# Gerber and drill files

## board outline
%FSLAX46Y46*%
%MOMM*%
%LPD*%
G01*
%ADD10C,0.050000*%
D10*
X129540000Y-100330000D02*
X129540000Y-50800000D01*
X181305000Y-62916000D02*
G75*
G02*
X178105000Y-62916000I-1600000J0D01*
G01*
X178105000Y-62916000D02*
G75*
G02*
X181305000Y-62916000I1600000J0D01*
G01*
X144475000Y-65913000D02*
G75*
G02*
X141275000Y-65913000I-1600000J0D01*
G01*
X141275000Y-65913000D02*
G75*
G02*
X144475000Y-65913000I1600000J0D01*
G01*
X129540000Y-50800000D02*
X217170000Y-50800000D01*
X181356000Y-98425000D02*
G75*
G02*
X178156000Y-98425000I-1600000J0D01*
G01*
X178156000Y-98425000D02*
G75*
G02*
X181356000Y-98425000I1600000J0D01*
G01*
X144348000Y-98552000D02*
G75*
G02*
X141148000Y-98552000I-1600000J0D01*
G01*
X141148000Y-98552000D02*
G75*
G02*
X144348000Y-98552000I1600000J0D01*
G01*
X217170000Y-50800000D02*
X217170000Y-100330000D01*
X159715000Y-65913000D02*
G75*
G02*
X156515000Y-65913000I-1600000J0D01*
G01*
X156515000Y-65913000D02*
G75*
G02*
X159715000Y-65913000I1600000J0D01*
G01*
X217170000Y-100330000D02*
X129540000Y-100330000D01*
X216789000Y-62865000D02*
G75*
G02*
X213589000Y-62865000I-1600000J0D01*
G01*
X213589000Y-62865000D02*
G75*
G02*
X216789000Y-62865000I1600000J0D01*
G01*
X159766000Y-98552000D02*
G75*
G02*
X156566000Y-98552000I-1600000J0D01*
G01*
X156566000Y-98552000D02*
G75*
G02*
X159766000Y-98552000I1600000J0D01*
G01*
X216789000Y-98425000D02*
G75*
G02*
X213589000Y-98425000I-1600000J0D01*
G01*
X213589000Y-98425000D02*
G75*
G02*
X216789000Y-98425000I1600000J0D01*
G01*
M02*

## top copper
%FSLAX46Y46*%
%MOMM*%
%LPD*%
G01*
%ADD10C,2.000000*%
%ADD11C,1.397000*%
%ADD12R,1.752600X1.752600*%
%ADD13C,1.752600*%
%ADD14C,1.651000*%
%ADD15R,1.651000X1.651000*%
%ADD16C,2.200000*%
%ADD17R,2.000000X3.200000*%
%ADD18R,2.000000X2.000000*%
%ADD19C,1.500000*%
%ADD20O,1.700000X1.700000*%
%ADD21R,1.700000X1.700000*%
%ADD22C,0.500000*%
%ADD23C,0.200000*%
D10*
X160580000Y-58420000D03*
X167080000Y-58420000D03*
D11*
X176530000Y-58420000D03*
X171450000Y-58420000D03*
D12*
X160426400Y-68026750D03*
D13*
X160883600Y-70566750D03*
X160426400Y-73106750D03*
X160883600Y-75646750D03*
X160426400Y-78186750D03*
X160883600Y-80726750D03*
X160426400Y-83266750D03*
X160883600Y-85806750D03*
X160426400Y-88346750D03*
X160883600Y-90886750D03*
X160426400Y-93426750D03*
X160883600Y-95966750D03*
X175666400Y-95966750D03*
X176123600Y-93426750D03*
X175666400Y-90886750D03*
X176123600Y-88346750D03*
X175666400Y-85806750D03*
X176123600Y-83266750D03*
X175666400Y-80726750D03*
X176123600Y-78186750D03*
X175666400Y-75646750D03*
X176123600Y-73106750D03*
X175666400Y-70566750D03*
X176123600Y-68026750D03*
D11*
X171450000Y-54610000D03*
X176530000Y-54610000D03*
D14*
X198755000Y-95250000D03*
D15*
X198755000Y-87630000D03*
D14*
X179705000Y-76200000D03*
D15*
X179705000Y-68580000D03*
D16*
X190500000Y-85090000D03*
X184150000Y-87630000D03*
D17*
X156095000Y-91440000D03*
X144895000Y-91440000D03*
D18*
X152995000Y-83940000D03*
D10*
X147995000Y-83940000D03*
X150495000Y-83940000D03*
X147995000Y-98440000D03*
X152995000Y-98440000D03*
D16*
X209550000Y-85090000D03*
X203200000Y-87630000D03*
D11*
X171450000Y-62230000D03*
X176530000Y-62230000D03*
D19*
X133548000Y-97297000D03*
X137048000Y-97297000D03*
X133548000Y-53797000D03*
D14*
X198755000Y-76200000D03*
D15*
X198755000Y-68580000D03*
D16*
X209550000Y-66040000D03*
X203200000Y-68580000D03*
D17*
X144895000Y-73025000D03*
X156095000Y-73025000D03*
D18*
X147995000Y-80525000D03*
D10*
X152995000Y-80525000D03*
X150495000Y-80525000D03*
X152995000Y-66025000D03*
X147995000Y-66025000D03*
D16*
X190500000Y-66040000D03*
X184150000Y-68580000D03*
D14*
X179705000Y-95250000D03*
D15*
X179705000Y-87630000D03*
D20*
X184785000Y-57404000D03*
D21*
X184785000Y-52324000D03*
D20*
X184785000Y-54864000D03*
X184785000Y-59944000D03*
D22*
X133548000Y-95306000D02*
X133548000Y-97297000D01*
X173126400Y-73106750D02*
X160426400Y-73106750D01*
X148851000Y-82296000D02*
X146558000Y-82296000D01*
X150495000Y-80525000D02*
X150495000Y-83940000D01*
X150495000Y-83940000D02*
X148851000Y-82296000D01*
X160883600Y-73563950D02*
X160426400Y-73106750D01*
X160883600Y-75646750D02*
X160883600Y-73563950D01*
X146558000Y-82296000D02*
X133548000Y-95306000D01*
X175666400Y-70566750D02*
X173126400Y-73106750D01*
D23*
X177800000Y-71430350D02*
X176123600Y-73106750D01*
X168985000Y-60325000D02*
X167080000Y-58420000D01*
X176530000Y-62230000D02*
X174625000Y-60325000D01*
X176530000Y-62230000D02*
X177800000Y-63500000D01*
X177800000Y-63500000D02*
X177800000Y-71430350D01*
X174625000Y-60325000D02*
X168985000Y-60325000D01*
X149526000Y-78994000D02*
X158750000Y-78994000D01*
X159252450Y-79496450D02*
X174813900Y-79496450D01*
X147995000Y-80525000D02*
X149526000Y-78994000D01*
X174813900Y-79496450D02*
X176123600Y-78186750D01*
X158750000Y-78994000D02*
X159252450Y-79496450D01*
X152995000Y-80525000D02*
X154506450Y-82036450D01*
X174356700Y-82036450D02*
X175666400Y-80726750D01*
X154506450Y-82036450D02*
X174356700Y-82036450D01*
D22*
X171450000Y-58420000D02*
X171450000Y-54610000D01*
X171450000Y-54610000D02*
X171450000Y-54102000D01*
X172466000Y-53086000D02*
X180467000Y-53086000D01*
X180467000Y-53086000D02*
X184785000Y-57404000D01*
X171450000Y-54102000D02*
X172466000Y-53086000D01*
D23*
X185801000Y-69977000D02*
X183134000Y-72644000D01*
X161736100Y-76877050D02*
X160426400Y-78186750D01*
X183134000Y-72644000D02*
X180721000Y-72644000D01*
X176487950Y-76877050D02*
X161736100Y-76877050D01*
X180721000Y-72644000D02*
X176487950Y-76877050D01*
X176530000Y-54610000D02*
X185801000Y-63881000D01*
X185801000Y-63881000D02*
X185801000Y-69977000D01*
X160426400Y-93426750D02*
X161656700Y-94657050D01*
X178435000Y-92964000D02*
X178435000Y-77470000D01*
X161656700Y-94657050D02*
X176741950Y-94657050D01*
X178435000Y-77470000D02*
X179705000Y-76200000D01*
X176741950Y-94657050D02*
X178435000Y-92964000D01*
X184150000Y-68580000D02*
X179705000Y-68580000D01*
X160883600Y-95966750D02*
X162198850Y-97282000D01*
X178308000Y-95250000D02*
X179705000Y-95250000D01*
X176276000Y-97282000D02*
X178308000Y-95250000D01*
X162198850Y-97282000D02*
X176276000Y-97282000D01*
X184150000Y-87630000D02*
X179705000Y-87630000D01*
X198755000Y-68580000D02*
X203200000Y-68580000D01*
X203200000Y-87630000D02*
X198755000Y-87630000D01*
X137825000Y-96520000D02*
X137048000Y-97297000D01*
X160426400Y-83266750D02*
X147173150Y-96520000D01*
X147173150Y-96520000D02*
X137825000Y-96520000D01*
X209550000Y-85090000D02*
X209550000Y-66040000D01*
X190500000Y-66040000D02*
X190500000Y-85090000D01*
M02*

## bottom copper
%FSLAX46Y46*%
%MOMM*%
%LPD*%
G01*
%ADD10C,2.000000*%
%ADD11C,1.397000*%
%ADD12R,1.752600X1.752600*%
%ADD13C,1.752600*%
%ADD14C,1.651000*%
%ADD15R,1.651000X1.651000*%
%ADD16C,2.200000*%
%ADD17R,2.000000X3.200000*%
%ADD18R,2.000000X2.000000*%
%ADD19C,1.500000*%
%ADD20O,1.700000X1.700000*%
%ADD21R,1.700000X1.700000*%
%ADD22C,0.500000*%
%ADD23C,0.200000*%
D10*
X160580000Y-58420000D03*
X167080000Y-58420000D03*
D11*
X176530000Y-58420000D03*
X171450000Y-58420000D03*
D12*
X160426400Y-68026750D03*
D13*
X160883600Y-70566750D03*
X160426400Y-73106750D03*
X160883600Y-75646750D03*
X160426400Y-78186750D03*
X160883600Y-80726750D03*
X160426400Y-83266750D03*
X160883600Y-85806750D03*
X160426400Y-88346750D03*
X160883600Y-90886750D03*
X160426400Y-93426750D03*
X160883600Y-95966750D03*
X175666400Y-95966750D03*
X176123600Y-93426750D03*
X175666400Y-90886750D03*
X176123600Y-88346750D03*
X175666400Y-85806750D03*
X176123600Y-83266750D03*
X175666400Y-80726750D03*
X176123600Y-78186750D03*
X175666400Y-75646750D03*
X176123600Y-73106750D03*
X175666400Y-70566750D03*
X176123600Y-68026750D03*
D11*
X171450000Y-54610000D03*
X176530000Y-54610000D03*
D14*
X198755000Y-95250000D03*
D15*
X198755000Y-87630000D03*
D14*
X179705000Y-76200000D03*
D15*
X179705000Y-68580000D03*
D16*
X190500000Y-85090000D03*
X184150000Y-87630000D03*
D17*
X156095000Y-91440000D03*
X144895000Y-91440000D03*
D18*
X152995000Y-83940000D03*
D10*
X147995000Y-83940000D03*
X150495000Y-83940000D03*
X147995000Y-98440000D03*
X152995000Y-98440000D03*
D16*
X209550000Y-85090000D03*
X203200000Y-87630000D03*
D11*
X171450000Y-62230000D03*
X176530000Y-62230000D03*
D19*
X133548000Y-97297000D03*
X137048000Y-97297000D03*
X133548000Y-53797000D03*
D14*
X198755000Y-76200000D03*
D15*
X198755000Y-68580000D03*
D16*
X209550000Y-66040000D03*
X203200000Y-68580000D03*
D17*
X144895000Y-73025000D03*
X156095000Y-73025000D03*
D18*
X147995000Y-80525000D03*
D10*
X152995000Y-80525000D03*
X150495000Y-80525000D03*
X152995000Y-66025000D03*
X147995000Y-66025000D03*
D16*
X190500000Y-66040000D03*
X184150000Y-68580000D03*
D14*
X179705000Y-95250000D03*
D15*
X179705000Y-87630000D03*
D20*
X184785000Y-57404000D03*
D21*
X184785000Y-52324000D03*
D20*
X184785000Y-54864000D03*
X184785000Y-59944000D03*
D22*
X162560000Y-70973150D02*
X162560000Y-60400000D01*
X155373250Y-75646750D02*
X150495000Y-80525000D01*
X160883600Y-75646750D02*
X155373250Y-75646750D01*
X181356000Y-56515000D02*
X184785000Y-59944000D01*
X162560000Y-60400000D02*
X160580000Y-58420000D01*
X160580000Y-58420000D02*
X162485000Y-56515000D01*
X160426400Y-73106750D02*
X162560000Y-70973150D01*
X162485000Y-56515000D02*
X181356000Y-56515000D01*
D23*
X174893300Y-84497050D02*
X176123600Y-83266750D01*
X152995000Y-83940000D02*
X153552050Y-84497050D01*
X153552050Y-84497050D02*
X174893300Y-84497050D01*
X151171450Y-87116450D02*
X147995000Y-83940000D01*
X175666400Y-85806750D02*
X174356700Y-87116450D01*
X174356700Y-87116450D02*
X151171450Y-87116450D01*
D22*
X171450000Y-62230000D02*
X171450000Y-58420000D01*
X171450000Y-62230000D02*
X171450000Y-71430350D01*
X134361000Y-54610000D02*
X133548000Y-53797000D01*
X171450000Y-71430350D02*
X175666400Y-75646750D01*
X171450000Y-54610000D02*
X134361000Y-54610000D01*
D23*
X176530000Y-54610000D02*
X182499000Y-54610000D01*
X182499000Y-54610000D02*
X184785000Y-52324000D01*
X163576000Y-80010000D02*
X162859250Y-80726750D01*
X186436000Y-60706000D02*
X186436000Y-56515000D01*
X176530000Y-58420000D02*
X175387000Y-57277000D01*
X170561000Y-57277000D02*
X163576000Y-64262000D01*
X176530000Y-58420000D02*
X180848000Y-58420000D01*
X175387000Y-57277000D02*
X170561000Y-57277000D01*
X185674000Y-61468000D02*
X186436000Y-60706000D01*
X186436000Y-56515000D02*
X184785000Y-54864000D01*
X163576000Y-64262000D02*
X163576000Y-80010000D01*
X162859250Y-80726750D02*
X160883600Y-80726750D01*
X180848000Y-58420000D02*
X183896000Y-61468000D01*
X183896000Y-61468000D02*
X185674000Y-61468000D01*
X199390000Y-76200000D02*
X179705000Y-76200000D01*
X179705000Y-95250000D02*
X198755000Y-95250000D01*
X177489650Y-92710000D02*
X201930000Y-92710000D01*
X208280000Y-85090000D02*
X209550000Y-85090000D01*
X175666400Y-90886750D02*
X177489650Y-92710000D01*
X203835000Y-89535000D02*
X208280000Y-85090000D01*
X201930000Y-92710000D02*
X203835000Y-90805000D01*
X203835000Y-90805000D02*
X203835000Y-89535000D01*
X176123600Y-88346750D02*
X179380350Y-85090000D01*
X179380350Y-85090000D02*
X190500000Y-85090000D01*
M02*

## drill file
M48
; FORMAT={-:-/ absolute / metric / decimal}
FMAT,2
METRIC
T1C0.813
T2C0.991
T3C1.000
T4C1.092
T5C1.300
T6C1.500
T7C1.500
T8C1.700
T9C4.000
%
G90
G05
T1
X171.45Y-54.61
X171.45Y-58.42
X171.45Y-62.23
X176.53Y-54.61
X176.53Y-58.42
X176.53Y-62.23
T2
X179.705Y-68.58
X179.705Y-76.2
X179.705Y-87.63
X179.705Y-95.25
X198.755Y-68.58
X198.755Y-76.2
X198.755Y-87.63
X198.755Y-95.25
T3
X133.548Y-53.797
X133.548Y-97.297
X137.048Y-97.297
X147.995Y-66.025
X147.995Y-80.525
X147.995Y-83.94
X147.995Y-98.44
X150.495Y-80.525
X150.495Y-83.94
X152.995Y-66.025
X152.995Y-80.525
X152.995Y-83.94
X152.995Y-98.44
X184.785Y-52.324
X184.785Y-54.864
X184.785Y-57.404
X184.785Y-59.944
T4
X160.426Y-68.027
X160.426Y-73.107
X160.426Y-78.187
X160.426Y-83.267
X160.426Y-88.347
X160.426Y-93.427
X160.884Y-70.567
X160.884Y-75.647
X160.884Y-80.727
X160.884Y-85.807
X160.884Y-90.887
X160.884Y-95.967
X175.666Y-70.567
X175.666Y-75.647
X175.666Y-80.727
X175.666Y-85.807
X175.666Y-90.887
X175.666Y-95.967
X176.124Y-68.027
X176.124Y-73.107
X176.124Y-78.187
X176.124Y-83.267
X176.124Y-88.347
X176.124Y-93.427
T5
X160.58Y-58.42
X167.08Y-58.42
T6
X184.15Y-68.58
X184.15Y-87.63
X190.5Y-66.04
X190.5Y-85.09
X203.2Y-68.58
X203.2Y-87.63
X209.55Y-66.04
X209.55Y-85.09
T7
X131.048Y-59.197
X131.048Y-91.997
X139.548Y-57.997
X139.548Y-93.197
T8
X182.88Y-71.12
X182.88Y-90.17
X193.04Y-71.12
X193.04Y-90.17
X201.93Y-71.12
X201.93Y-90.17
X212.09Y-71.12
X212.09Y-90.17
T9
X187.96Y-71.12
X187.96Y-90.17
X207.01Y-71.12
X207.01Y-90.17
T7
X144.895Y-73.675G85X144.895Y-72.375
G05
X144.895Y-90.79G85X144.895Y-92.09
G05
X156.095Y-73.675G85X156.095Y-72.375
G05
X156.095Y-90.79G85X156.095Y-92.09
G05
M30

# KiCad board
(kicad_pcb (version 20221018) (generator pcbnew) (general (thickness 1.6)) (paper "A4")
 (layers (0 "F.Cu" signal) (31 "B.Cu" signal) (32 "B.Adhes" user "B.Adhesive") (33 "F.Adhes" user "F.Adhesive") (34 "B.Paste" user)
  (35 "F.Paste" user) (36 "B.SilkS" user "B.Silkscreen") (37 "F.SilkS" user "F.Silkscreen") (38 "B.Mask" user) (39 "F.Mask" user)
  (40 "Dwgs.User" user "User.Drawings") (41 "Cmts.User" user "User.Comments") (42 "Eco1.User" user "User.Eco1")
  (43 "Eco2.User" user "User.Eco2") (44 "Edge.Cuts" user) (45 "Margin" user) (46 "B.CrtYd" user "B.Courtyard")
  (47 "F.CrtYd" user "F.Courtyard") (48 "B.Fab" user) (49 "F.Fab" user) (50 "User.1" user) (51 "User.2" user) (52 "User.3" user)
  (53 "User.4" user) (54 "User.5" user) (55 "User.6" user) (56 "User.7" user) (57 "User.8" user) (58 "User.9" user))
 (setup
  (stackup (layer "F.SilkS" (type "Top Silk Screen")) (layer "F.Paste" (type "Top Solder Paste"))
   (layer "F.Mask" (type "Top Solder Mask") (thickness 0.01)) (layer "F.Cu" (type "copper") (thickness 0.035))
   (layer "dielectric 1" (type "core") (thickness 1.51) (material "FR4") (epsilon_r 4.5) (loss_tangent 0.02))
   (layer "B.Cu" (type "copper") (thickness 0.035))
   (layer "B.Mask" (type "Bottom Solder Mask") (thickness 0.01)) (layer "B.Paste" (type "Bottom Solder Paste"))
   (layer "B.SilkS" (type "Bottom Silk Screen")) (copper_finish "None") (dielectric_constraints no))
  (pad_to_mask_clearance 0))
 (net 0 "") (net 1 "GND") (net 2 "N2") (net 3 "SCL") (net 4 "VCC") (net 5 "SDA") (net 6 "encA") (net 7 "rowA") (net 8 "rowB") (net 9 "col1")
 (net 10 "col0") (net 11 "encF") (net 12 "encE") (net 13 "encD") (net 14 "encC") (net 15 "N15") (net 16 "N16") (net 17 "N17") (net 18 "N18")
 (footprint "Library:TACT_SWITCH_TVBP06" (layer "F.Cu") (at 163.83 58.42)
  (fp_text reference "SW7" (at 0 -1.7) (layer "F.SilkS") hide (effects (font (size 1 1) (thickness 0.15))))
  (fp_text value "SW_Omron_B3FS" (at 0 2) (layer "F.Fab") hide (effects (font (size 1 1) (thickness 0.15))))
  (pad "1" thru_hole circle (at -3.25 0) (size 2 2) (drill 1.3) (layers "*.Cu" "*.Mask") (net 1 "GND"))
  (pad "2" thru_hole circle (at 3.25 0) (size 2 2) (drill 1.3) (layers "*.Cu" "*.Mask") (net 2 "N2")))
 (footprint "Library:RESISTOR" (layer "F.Cu") (at 173.99 58.42 180)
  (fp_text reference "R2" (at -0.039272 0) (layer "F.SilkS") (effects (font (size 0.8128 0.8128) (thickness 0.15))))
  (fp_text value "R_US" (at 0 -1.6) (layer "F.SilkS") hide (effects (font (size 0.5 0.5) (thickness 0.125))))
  (pad "1" thru_hole circle (at -2.54 0 180) (size 1.397 1.397) (drill 0.8128) (layers "*.Cu" "*.Mask") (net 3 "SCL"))
  (pad "2" thru_hole circle (at 2.54 0 180) (size 1.397 1.397) (drill 0.8128) (layers "*.Cu" "*.Mask") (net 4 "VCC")))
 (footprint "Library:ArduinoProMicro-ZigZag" (layer "F.Cu") (at 168.275 81.99675 -90)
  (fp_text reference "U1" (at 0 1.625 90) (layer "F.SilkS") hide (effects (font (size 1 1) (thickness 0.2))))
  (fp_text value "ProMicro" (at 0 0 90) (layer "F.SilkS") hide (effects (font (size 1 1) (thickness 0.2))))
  (pad "1" thru_hole rect (at -13.97 7.8486 270) (size 1.7526 1.7526) (drill 1.0922) (layers "*.Cu" "*.SilkS" "*.Mask"))
  (pad "2" thru_hole circle (at -11.43 7.3914 270) (size 1.7526 1.7526) (drill 1.0922) (layers "*.Cu" "*.SilkS" "*.Mask"))
  (pad "3" thru_hole circle (at -8.89 7.8486 270) (size 1.7526 1.7526) (drill 1.0922) (layers "*.Cu" "*.SilkS" "*.Mask") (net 1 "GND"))
  (pad "4" thru_hole circle (at -6.35 7.3914 270) (size 1.7526 1.7526) (drill 1.0922) (layers "*.Cu" "*.SilkS" "*.Mask") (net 1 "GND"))
  (pad "5" thru_hole circle (at -3.81 7.8486 270) (size 1.7526 1.7526) (drill 1.0922) (layers "*.Cu" "*.SilkS" "*.Mask") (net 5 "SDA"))
  (pad "6" thru_hole circle (at -1.27 7.3914 270) (size 1.7526 1.7526) (drill 1.0922) (layers "*.Cu" "*.SilkS" "*.Mask") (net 3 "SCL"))
  (pad "7" thru_hole circle (at 1.27 7.8486 270) (size 1.7526 1.7526) (drill 1.0922) (layers "*.Cu" "*.SilkS" "*.Mask") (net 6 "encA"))
  (pad "8" thru_hole circle (at 3.81 7.3914 270) (size 1.7526 1.7526) (drill 1.0922) (layers "*.Cu" "*.SilkS" "*.Mask"))
  (pad "9" thru_hole circle (at 6.35 7.8486 270) (size 1.7526 1.7526) (drill 1.0922) (layers "*.Cu" "*.SilkS" "*.Mask"))
  (pad "10" thru_hole circle (at 8.89 7.3914 270) (size 1.7526 1.7526) (drill 1.0922) (layers "*.Cu" "*.SilkS" "*.Mask"))
  (pad "11" thru_hole circle (at 11.43 7.8486 270) (size 1.7526 1.7526) (drill 1.0922) (layers "*.Cu" "*.SilkS" "*.Mask") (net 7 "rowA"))
  (pad "12" thru_hole circle (at 13.97 7.3914 270) (size 1.7526 1.7526) (drill 1.0922) (layers "*.Cu" "*.SilkS" "*.Mask") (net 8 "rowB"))
  (pad "13" thru_hole circle (at 13.97 -7.3914 270) (size 1.7526 1.7526) (drill 1.0922) (layers "*.Cu" "*.SilkS" "*.Mask"))
  (pad "14" thru_hole circle (at 11.43 -7.8486 270) (size 1.7526 1.7526) (drill 1.0922) (layers "*.Cu" "*.SilkS" "*.Mask"))
  (pad "15" thru_hole circle (at 8.89 -7.3914 270) (size 1.7526 1.7526) (drill 1.0922) (layers "*.Cu" "*.SilkS" "*.Mask") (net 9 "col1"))
  (pad "16" thru_hole circle (at 6.35 -7.8486 270) (size 1.7526 1.7526) (drill 1.0922) (layers "*.Cu" "*.SilkS" "*.Mask") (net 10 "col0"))
  (pad "17" thru_hole circle (at 3.81 -7.3914 270) (size 1.7526 1.7526) (drill 1.0922) (layers "*.Cu" "*.SilkS" "*.Mask") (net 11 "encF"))
  (pad "18" thru_hole circle (at 1.27 -7.8486 270) (size 1.7526 1.7526) (drill 1.0922) (layers "*.Cu" "*.SilkS" "*.Mask") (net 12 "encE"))
  (pad "19" thru_hole circle (at -1.27 -7.3914 270) (size 1.7526 1.7526) (drill 1.0922) (layers "*.Cu" "*.SilkS" "*.Mask") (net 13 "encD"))
  (pad "20" thru_hole circle (at -3.81 -7.8486 270) (size 1.7526 1.7526) (drill 1.0922) (layers "*.Cu" "*.SilkS" "*.Mask") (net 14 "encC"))
  (pad "21" thru_hole circle (at -6.35 -7.3914 270) (size 1.7526 1.7526) (drill 1.0922) (layers "*.Cu" "*.SilkS" "*.Mask") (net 4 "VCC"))
  (pad "22" thru_hole circle (at -8.89 -7.8486 270) (size 1.7526 1.7526) (drill 1.0922) (layers "*.Cu" "*.SilkS" "*.Mask") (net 2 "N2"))
  (pad "23" thru_hole circle (at -11.43 -7.3914 270) (size 1.7526 1.7526) (drill 1.0922) (layers "*.Cu" "*.SilkS" "*.Mask") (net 1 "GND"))
  (pad "24" thru_hole circle (at -13.97 -7.8486 270) (size 1.7526 1.7526) (drill 1.0922) (layers "*.Cu" "*.SilkS" "*.Mask")))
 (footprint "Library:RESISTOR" (layer "F.Cu") (at 173.99 54.61)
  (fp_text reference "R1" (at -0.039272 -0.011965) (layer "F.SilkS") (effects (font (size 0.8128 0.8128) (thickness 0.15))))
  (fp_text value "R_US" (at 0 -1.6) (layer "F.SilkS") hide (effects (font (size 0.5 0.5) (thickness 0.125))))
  (pad "1" thru_hole circle (at -2.54 0) (size 1.397 1.397) (drill 0.8128) (layers "*.Cu" "*.Mask") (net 4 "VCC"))
  (pad "2" thru_hole circle (at 2.54 0) (size 1.397 1.397) (drill 0.8128) (layers "*.Cu" "*.Mask") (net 5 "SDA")))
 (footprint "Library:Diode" (layer "F.Cu") (at 198.755 91.44 90)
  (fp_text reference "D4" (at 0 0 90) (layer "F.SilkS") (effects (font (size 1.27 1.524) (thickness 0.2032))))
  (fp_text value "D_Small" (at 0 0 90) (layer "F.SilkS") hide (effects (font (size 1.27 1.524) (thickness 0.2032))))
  (pad "1" thru_hole circle (at -3.81 0 90) (size 1.651 1.651) (drill 0.9906) (layers "*.Cu" "*.SilkS" "*.Mask") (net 8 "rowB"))
  (pad "2" thru_hole rect (at 3.81 0 90) (size 1.651 1.651) (drill 0.9906) (layers "*.Cu" "*.SilkS" "*.Mask") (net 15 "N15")))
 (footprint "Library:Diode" (layer "F.Cu") (at 179.705 72.39 90)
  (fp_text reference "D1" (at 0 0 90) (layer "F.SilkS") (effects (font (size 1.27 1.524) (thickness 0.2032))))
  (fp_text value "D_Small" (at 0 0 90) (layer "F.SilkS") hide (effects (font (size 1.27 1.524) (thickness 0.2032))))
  (pad "1" thru_hole circle (at -3.81 0 90) (size 1.651 1.651) (drill 0.9906) (layers "*.Cu" "*.SilkS" "*.Mask") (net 7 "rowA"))
  (pad "2" thru_hole rect (at 3.81 0 90) (size 1.651 1.651) (drill 0.9906) (layers "*.Cu" "*.SilkS" "*.Mask") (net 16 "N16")))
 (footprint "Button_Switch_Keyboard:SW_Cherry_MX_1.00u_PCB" (layer "F.Cu") (at 190.5 85.09)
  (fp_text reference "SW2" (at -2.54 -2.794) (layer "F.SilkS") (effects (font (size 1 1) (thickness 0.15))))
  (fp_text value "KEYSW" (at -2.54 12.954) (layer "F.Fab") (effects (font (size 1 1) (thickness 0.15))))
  (pad "" np_thru_hole circle (at -7.62 5.08) (size 1.7 1.7) (drill 1.7) (layers "*.Cu" "*.Mask"))
  (pad "" np_thru_hole circle (at -2.54 5.08) (size 4 4) (drill 4) (layers "*.Cu" "*.Mask"))
  (pad "" np_thru_hole circle (at 2.54 5.08) (size 1.7 1.7) (drill 1.7) (layers "*.Cu" "*.Mask"))
  (pad "1" thru_hole circle (at 0 0) (size 2.2 2.2) (drill 1.5) (layers "*.Cu" "*.Mask") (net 10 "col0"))
  (pad "2" thru_hole circle (at -6.35 2.54) (size 2.2 2.2) (drill 1.5) (layers "*.Cu" "*.Mask") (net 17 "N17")))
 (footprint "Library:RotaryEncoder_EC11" (layer "F.Cu") (at 150.495 91.44 -90)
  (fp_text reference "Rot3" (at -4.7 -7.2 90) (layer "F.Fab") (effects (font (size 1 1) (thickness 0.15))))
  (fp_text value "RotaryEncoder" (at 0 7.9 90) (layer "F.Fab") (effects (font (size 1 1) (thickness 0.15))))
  (pad "" np_thru_hole rect (at 0 -5.6 270) (size 3.2 2) (drill oval 2.8 1.5) (layers "*.Cu" "*.Mask"))
  (pad "" np_thru_hole rect (at 0 5.6 270) (size 3.2 2) (drill oval 2.8 1.5) (layers "*.Cu" "*.Mask"))
  (pad "A" thru_hole rect (at -7.5 -2.5 270) (size 2 2) (drill 1) (layers "*.Cu" "*.Mask") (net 12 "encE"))
  (pad "B" thru_hole circle (at -7.5 2.5 270) (size 2 2) (drill 1) (layers "*.Cu" "*.Mask") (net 11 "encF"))
  (pad "C" thru_hole circle (at -7.5 0 270) (size 2 2) (drill 1) (layers "*.Cu" "*.Mask") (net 1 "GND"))
  (pad "S1" thru_hole circle (at 7 2.5 270) (size 2 2) (drill 1) (layers "*.Cu" "*.Mask"))
  (pad "S2" thru_hole circle (at 7 -2.5 270) (size 2 2) (drill 1) (layers "*.Cu" "*.Mask")))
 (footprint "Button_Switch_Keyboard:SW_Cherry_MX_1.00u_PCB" (layer "F.Cu") (at 209.55 85.09)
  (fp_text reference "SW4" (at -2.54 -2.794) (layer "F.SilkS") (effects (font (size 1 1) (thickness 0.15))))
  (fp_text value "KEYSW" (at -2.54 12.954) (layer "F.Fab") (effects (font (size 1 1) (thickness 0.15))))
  (pad "" np_thru_hole circle (at -7.62 5.08) (size 1.7 1.7) (drill 1.7) (layers "*.Cu" "*.Mask"))
  (pad "" np_thru_hole circle (at -2.54 5.08) (size 4 4) (drill 4) (layers "*.Cu" "*.Mask"))
  (pad "" np_thru_hole circle (at 2.54 5.08) (size 1.7 1.7) (drill 1.7) (layers "*.Cu" "*.Mask"))
  (pad "1" thru_hole circle (at 0 0) (size 2.2 2.2) (drill 1.5) (layers "*.Cu" "*.Mask") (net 9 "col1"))
  (pad "2" thru_hole circle (at -6.35 2.54) (size 2.2 2.2) (drill 1.5) (layers "*.Cu" "*.Mask") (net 15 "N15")))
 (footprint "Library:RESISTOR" (layer "F.Cu") (at 173.99 62.23)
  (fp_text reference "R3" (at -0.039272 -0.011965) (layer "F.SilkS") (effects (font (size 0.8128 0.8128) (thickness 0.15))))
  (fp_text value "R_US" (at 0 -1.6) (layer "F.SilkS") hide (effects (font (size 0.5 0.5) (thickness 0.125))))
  (pad "1" thru_hole circle (at -2.54 0) (size 1.397 1.397) (drill 0.8128) (layers "*.Cu" "*.Mask") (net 4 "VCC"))
  (pad "2" thru_hole circle (at 2.54 0) (size 1.397 1.397) (drill 0.8128) (layers "*.Cu" "*.Mask") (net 2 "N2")))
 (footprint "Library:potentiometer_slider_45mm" (layer "F.Cu") (at 142.248 98.097 90)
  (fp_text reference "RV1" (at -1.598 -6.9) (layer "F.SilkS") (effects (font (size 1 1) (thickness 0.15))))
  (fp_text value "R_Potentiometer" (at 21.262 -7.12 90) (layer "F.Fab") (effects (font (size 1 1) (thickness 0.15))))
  (pad "" np_thru_hole circle (at 4.9 -2.7 90) (size 1.5 1.5) (drill 1.5) (layers "*.Cu" "*.Mask"))
  (pad "" np_thru_hole circle (at 6.1 -11.2 90) (size 1.5 1.5) (drill 1.5) (layers "*.Cu" "*.Mask"))
  (pad "" np_thru_hole circle (at 38.9 -11.2 90) (size 1.5 1.5) (drill 1.5) (layers "*.Cu" "*.Mask"))
  (pad "" np_thru_hole circle (at 40.1 -2.7 90) (size 1.5 1.5) (drill 1.5) (layers "*.Cu" "*.Mask"))
  (pad "1" thru_hole circle (at 0.8 -8.7 90) (size 1.5 1.5) (drill 1) (layers "*.Cu" "*.Mask") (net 1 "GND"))
  (pad "2" thru_hole circle (at 0.8 -5.2 90) (size 1.5 1.5) (drill 1) (layers "*.Cu" "*.Mask") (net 6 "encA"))
  (pad "3" thru_hole circle (at 44.3 -8.7 90) (size 1.5 1.5) (drill 1) (layers "*.Cu" "*.Mask") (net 4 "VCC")))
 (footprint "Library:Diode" (layer "F.Cu") (at 198.755 72.39 90)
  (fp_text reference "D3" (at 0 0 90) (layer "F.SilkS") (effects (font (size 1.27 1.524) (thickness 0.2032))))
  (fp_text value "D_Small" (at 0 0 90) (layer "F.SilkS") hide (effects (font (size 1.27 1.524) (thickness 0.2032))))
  (pad "1" thru_hole circle (at -3.81 0 90) (size 1.651 1.651) (drill 0.9906) (layers "*.Cu" "*.SilkS" "*.Mask") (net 7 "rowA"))
  (pad "2" thru_hole rect (at 3.81 0 90) (size 1.651 1.651) (drill 0.9906) (layers "*.Cu" "*.SilkS" "*.Mask") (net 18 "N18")))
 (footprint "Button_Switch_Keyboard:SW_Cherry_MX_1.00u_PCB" (layer "F.Cu") (at 209.55 66.04)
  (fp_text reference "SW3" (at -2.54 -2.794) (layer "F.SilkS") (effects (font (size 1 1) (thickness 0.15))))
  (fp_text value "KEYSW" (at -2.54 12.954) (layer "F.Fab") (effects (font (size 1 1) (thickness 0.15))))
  (pad "" np_thru_hole circle (at -7.62 5.08) (size 1.7 1.7) (drill 1.7) (layers "*.Cu" "*.Mask"))
  (pad "" np_thru_hole circle (at -2.54 5.08) (size 4 4) (drill 4) (layers "*.Cu" "*.Mask"))
  (pad "" np_thru_hole circle (at 2.54 5.08) (size 1.7 1.7) (drill 1.7) (layers "*.Cu" "*.Mask"))
  (pad "1" thru_hole circle (at 0 0) (size 2.2 2.2) (drill 1.5) (layers "*.Cu" "*.Mask") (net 9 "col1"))
  (pad "2" thru_hole circle (at -6.35 2.54) (size 2.2 2.2) (drill 1.5) (layers "*.Cu" "*.Mask") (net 18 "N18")))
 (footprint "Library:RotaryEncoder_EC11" (layer "F.Cu") (at 150.495 73.025 90)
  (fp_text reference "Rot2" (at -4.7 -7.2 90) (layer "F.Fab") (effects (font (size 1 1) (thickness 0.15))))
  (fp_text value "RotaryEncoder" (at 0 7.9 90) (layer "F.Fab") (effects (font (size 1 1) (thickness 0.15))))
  (pad "" np_thru_hole rect (at 0 -5.6 90) (size 3.2 2) (drill oval 2.8 1.5) (layers "*.Cu" "*.Mask"))
  (pad "" np_thru_hole rect (at 0 5.6 90) (size 3.2 2) (drill oval 2.8 1.5) (layers "*.Cu" "*.Mask"))
  (pad "A" thru_hole rect (at -7.5 -2.5 90) (size 2 2) (drill 1) (layers "*.Cu" "*.Mask") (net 14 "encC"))
  (pad "B" thru_hole circle (at -7.5 2.5 90) (size 2 2) (drill 1) (layers "*.Cu" "*.Mask") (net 13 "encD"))
  (pad "C" thru_hole circle (at -7.5 0 90) (size 2 2) (drill 1) (layers "*.Cu" "*.Mask") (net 1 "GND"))
  (pad "S1" thru_hole circle (at 7 2.5 90) (size 2 2) (drill 1) (layers "*.Cu" "*.Mask"))
  (pad "S2" thru_hole circle (at 7 -2.5 90) (size 2 2) (drill 1) (layers "*.Cu" "*.Mask")))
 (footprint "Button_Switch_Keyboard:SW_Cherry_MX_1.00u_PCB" (layer "F.Cu") (at 190.5 66.04)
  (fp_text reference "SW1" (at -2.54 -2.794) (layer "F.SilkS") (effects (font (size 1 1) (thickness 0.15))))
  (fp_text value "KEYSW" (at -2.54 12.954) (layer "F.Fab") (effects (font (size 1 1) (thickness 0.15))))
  (pad "" np_thru_hole circle (at -7.62 5.08) (size 1.7 1.7) (drill 1.7) (layers "*.Cu" "*.Mask"))
  (pad "" np_thru_hole circle (at -2.54 5.08) (size 4 4) (drill 4) (layers "*.Cu" "*.Mask"))
  (pad "" np_thru_hole circle (at 2.54 5.08) (size 1.7 1.7) (drill 1.7) (layers "*.Cu" "*.Mask"))
  (pad "1" thru_hole circle (at 0 0) (size 2.2 2.2) (drill 1.5) (layers "*.Cu" "*.Mask") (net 10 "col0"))
  (pad "2" thru_hole circle (at -6.35 2.54) (size 2.2 2.2) (drill 1.5) (layers "*.Cu" "*.Mask") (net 16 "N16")))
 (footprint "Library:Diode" (layer "F.Cu") (at 179.705 91.44 90)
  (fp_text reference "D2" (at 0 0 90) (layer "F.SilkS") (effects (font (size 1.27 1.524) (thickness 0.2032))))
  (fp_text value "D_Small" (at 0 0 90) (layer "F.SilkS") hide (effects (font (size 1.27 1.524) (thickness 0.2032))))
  (pad "1" thru_hole circle (at -3.81 0 90) (size 1.651 1.651) (drill 0.9906) (layers "*.Cu" "*.SilkS" "*.Mask") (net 8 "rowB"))
  (pad "2" thru_hole rect (at 3.81 0 90) (size 1.651 1.651) (drill 0.9906) (layers "*.Cu" "*.SilkS" "*.Mask") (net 17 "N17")))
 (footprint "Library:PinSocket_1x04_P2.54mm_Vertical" (layer "F.Cu") (at 184.785 52.324)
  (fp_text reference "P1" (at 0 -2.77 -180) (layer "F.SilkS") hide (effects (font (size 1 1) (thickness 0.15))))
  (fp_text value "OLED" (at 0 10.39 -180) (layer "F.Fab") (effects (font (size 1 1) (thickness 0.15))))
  (pad "" thru_hole oval (at 0 5.08) (size 1.7 1.7) (drill 1) (layers "*.Cu" "*.Mask") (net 4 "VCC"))
  (pad "1" thru_hole rect (at 0 0) (size 1.7 1.7) (drill 1) (layers "*.Cu" "*.Mask") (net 5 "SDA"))
  (pad "2" thru_hole oval (at 0 2.54) (size 1.7 1.7) (drill 1) (layers "*.Cu" "*.Mask") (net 3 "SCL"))
  (pad "4" thru_hole oval (at 0 7.62) (size 1.7 1.7) (drill 1) (layers "*.Cu" "*.Mask") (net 1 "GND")))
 (gr_line (start 129.54 100.33) (end 129.54 50.8) (stroke (width 0.05) (type default)) (layer "Edge.Cuts"))
 (gr_circle (center 179.705 62.916) (end 181.305 62.916) (stroke (width 0.05) (type default)) (fill none) (layer "Edge.Cuts"))
 (gr_circle (center 142.875 65.913) (end 144.475 65.913) (stroke (width 0.05) (type default)) (fill none) (layer "Edge.Cuts"))
 (gr_line (start 129.54 50.8) (end 217.17 50.8) (stroke (width 0.05) (type default)) (layer "Edge.Cuts"))
 (gr_circle (center 179.756 98.425) (end 181.356 98.425) (stroke (width 0.05) (type default)) (fill none) (layer "Edge.Cuts"))
 (gr_circle (center 142.748 98.552) (end 144.348 98.552) (stroke (width 0.05) (type default)) (fill none) (layer "Edge.Cuts"))
 (gr_line (start 217.17 50.8) (end 217.17 100.33) (stroke (width 0.05) (type default)) (layer "Edge.Cuts"))
 (gr_circle (center 158.115 65.913) (end 159.715 65.913) (stroke (width 0.05) (type default)) (fill none) (layer "Edge.Cuts"))
 (gr_line (start 217.17 100.33) (end 129.54 100.33) (stroke (width 0.05) (type default)) (layer "Edge.Cuts"))
 (gr_circle (center 215.189 62.865) (end 216.789 62.865) (stroke (width 0.05) (type default)) (fill none) (layer "Edge.Cuts"))
 (gr_circle (center 158.166 98.552) (end 159.766 98.552) (stroke (width 0.05) (type default)) (fill none) (layer "Edge.Cuts"))
 (gr_circle (center 215.189 98.425) (end 216.789 98.425) (stroke (width 0.05) (type default)) (fill none) (layer "Edge.Cuts"))
 (segment (start 133.548 95.306) (end 133.548 97.297) (width 0.5) (layer "F.Cu") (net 1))
 (segment (start 173.1264 73.10675) (end 160.4264 73.10675) (width 0.5) (layer "F.Cu") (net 1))
 (segment (start 148.851 82.296) (end 146.558 82.296) (width 0.5) (layer "F.Cu") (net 1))
 (segment (start 150.495 80.525) (end 150.495 83.94) (width 0.5) (layer "F.Cu") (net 1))
 (segment (start 150.495 83.94) (end 148.851 82.296) (width 0.5) (layer "F.Cu") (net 1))
 (segment (start 160.8836 73.56395) (end 160.4264 73.10675) (width 0.5) (layer "F.Cu") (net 1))
 (segment (start 160.8836 75.64675) (end 160.8836 73.56395) (width 0.5) (layer "F.Cu") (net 1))
 (segment (start 146.558 82.296) (end 133.548 95.306) (width 0.5) (layer "F.Cu") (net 1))
 (segment (start 175.6664 70.56675) (end 173.1264 73.10675) (width 0.5) (layer "F.Cu") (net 1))
 (segment (start 162.56 70.97315) (end 162.56 60.4) (width 0.5) (layer "B.Cu") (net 1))
 (segment (start 155.37325 75.64675) (end 150.495 80.525) (width 0.5) (layer "B.Cu") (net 1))
 (segment (start 160.8836 75.64675) (end 155.37325 75.64675) (width 0.5) (layer "B.Cu") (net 1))
 (segment (start 181.356 56.515) (end 184.785 59.944) (width 0.5) (layer "B.Cu") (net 1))
 (segment (start 162.56 60.4) (end 160.58 58.42) (width 0.5) (layer "B.Cu") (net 1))
 (segment (start 160.58 58.42) (end 162.485 56.515) (width 0.5) (layer "B.Cu") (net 1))
 (segment (start 160.4264 73.10675) (end 162.56 70.97315) (width 0.5) (layer "B.Cu") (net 1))
 (segment (start 162.485 56.515) (end 181.356 56.515) (width 0.5) (layer "B.Cu") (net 1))
 (segment (start 177.8 71.43035) (end 176.1236 73.10675) (width 0.2) (layer "F.Cu") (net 2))
 (segment (start 168.985 60.325) (end 167.08 58.42) (width 0.2) (layer "F.Cu") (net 2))
 (segment (start 176.53 62.23) (end 174.625 60.325) (width 0.2) (layer "F.Cu") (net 2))
 (segment (start 176.53 62.23) (end 177.8 63.5) (width 0.2) (layer "F.Cu") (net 2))
 (segment (start 177.8 63.5) (end 177.8 71.43035) (width 0.2) (layer "F.Cu") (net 2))
 (segment (start 174.625 60.325) (end 168.985 60.325) (width 0.2) (layer "F.Cu") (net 2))
 (segment (start 149.526 78.994) (end 158.75 78.994) (width 0.2) (layer "F.Cu") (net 14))
 (segment (start 159.25245 79.49645) (end 174.8139 79.49645) (width 0.2) (layer "F.Cu") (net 14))
 (segment (start 147.995 80.525) (end 149.526 78.994) (width 0.2) (layer "F.Cu") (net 14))
 (segment (start 174.8139 79.49645) (end 176.1236 78.18675) (width 0.2) (layer "F.Cu") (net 14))
 (segment (start 158.75 78.994) (end 159.25245 79.49645) (width 0.2) (layer "F.Cu") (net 14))
 (segment (start 152.995 80.525) (end 154.50645 82.03645) (width 0.2) (layer "F.Cu") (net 13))
 (segment (start 174.3567 82.03645) (end 175.6664 80.72675) (width 0.2) (layer "F.Cu") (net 13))
 (segment (start 154.50645 82.03645) (end 174.3567 82.03645) (width 0.2) (layer "F.Cu") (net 13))
 (segment (start 174.8933 84.49705) (end 176.1236 83.26675) (width 0.2) (layer "B.Cu") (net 12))
 (segment (start 152.995 83.94) (end 153.55205 84.49705) (width 0.2) (layer "B.Cu") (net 12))
 (segment (start 153.55205 84.49705) (end 174.8933 84.49705) (width 0.2) (layer "B.Cu") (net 12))
 (segment (start 151.17145 87.11645) (end 147.995 83.94) (width 0.2) (layer "B.Cu") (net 11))
 (segment (start 175.6664 85.80675) (end 174.3567 87.11645) (width 0.2) (layer "B.Cu") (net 11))
 (segment (start 174.3567 87.11645) (end 151.17145 87.11645) (width 0.2) (layer "B.Cu") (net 11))
 (segment (start 171.45 58.42) (end 171.45 54.61) (width 0.5) (layer "F.Cu") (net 4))
 (segment (start 171.45 54.61) (end 171.45 54.102) (width 0.5) (layer "F.Cu") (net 4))
 (segment (start 172.466 53.086) (end 180.467 53.086) (width 0.5) (layer "F.Cu") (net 4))
 (segment (start 180.467 53.086) (end 184.785 57.404) (width 0.5) (layer "F.Cu") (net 4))
 (segment (start 171.45 54.102) (end 172.466 53.086) (width 0.5) (layer "F.Cu") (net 4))
 (segment (start 171.45 62.23) (end 171.45 58.42) (width 0.5) (layer "B.Cu") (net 4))
 (segment (start 171.45 62.23) (end 171.45 71.43035) (width 0.5) (layer "B.Cu") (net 4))
 (segment (start 134.361 54.61) (end 133.548 53.797) (width 0.5) (layer "B.Cu") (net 4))
 (segment (start 171.45 71.43035) (end 175.6664 75.64675) (width 0.5) (layer "B.Cu") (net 4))
 (segment (start 171.45 54.61) (end 134.361 54.61) (width 0.5) (layer "B.Cu") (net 4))
 (segment (start 185.801 69.977) (end 183.134 72.644) (width 0.2) (layer "F.Cu") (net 5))
 (segment (start 161.7361 76.87705) (end 160.4264 78.18675) (width 0.2) (layer "F.Cu") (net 5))
 (segment (start 183.134 72.644) (end 180.721 72.644) (width 0.2) (layer "F.Cu") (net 5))
 (segment (start 176.48795 76.87705) (end 161.7361 76.87705) (width 0.2) (layer "F.Cu") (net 5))
 (segment (start 180.721 72.644) (end 176.48795 76.87705) (width 0.2) (layer "F.Cu") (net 5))
 (segment (start 176.53 54.61) (end 185.801 63.881) (width 0.2) (layer "F.Cu") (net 5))
 (segment (start 185.801 63.881) (end 185.801 69.977) (width 0.2) (layer "F.Cu") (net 5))
 (segment (start 176.53 54.61) (end 182.499 54.61) (width 0.2) (layer "B.Cu") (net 5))
 (segment (start 182.499 54.61) (end 184.785 52.324) (width 0.2) (layer "B.Cu") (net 5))
 (segment (start 163.576 80.01) (end 162.85925 80.72675) (width 0.2) (layer "B.Cu") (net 3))
 (segment (start 186.436 60.706) (end 186.436 56.515) (width 0.2) (layer "B.Cu") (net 3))
 (segment (start 176.53 58.42) (end 175.387 57.277) (width 0.2) (layer "B.Cu") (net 3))
 (segment (start 170.561 57.277) (end 163.576 64.262) (width 0.2) (layer "B.Cu") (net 3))
 (segment (start 176.53 58.42) (end 180.848 58.42) (width 0.2) (layer "B.Cu") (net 3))
 (segment (start 175.387 57.277) (end 170.561 57.277) (width 0.2) (layer "B.Cu") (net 3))
 (segment (start 185.674 61.468) (end 186.436 60.706) (width 0.2) (layer "B.Cu") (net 3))
 (segment (start 186.436 56.515) (end 184.785 54.864) (width 0.2) (layer "B.Cu") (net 3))
 (segment (start 163.576 64.262) (end 163.576 80.01) (width 0.2) (layer "B.Cu") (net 3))
 (segment (start 162.85925 80.72675) (end 160.8836 80.72675) (width 0.2) (layer "B.Cu") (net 3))
 (segment (start 180.848 58.42) (end 183.896 61.468) (width 0.2) (layer "B.Cu") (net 3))
 (segment (start 183.896 61.468) (end 185.674 61.468) (width 0.2) (layer "B.Cu") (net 3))
 (segment (start 160.4264 93.42675) (end 161.6567 94.65705) (width 0.2) (layer "F.Cu") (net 7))
 (segment (start 178.435 92.964) (end 178.435 77.47) (width 0.2) (layer "F.Cu") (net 7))
 (segment (start 161.6567 94.65705) (end 176.74195 94.65705) (width 0.2) (layer "F.Cu") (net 7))
 (segment (start 178.435 77.47) (end 179.705 76.2) (width 0.2) (layer "F.Cu") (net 7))
 (segment (start 176.74195 94.65705) (end 178.435 92.964) (width 0.2) (layer "F.Cu") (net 7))
 (segment (start 199.39 76.2) (end 179.705 76.2) (width 0.2) (layer "B.Cu") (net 7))
 (segment (start 184.15 68.58) (end 179.705 68.58) (width 0.2) (layer "F.Cu") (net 16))
 (segment (start 160.8836 95.96675) (end 162.19885 97.282) (width 0.2) (layer "F.Cu") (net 8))
 (segment (start 178.308 95.25) (end 179.705 95.25) (width 0.2) (layer "F.Cu") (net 8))
 (segment (start 176.276 97.282) (end 178.308 95.25) (width 0.2) (layer "F.Cu") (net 8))
 (segment (start 162.19885 97.282) (end 176.276 97.282) (width 0.2) (layer "F.Cu") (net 8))
 (segment (start 179.705 95.25) (end 198.755 95.25) (width 0.2) (layer "B.Cu") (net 8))
 (segment (start 184.15 87.63) (end 179.705 87.63) (width 0.2) (layer "F.Cu") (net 17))
 (segment (start 198.755 68.58) (end 203.2 68.58) (width 0.2) (layer "F.Cu") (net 18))
 (segment (start 203.2 87.63) (end 198.755 87.63) (width 0.2) (layer "F.Cu") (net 15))
 (segment (start 137.825 96.52) (end 137.048 97.297) (width 0.2) (layer "F.Cu") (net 6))
 (segment (start 160.4264 83.26675) (end 147.17315 96.52) (width 0.2) (layer "F.Cu") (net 6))
 (segment (start 147.17315 96.52) (end 137.825 96.52) (width 0.2) (layer "F.Cu") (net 6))
 (segment (start 209.55 85.09) (end 209.55 66.04) (width 0.2) (layer "F.Cu") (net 9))
 (segment (start 177.48965 92.71) (end 201.93 92.71) (width 0.2) (layer "B.Cu") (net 9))
 (segment (start 208.28 85.09) (end 209.55 85.09) (width 0.2) (layer "B.Cu") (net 9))
 (segment (start 175.6664 90.88675) (end 177.48965 92.71) (width 0.2) (layer "B.Cu") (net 9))
 (segment (start 203.835 89.535) (end 208.28 85.09) (width 0.2) (layer "B.Cu") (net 9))
 (segment (start 201.93 92.71) (end 203.835 90.805) (width 0.2) (layer "B.Cu") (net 9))
 (segment (start 203.835 90.805) (end 203.835 89.535) (width 0.2) (layer "B.Cu") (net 9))
 (segment (start 190.5 66.04) (end 190.5 85.09) (width 0.2) (layer "F.Cu") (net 10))
 (segment (start 176.1236 88.34675) (end 179.38035 85.09) (width 0.2) (layer "B.Cu") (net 10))
 (segment (start 179.38035 85.09) (end 190.5 85.09) (width 0.2) (layer "B.Cu") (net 10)))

